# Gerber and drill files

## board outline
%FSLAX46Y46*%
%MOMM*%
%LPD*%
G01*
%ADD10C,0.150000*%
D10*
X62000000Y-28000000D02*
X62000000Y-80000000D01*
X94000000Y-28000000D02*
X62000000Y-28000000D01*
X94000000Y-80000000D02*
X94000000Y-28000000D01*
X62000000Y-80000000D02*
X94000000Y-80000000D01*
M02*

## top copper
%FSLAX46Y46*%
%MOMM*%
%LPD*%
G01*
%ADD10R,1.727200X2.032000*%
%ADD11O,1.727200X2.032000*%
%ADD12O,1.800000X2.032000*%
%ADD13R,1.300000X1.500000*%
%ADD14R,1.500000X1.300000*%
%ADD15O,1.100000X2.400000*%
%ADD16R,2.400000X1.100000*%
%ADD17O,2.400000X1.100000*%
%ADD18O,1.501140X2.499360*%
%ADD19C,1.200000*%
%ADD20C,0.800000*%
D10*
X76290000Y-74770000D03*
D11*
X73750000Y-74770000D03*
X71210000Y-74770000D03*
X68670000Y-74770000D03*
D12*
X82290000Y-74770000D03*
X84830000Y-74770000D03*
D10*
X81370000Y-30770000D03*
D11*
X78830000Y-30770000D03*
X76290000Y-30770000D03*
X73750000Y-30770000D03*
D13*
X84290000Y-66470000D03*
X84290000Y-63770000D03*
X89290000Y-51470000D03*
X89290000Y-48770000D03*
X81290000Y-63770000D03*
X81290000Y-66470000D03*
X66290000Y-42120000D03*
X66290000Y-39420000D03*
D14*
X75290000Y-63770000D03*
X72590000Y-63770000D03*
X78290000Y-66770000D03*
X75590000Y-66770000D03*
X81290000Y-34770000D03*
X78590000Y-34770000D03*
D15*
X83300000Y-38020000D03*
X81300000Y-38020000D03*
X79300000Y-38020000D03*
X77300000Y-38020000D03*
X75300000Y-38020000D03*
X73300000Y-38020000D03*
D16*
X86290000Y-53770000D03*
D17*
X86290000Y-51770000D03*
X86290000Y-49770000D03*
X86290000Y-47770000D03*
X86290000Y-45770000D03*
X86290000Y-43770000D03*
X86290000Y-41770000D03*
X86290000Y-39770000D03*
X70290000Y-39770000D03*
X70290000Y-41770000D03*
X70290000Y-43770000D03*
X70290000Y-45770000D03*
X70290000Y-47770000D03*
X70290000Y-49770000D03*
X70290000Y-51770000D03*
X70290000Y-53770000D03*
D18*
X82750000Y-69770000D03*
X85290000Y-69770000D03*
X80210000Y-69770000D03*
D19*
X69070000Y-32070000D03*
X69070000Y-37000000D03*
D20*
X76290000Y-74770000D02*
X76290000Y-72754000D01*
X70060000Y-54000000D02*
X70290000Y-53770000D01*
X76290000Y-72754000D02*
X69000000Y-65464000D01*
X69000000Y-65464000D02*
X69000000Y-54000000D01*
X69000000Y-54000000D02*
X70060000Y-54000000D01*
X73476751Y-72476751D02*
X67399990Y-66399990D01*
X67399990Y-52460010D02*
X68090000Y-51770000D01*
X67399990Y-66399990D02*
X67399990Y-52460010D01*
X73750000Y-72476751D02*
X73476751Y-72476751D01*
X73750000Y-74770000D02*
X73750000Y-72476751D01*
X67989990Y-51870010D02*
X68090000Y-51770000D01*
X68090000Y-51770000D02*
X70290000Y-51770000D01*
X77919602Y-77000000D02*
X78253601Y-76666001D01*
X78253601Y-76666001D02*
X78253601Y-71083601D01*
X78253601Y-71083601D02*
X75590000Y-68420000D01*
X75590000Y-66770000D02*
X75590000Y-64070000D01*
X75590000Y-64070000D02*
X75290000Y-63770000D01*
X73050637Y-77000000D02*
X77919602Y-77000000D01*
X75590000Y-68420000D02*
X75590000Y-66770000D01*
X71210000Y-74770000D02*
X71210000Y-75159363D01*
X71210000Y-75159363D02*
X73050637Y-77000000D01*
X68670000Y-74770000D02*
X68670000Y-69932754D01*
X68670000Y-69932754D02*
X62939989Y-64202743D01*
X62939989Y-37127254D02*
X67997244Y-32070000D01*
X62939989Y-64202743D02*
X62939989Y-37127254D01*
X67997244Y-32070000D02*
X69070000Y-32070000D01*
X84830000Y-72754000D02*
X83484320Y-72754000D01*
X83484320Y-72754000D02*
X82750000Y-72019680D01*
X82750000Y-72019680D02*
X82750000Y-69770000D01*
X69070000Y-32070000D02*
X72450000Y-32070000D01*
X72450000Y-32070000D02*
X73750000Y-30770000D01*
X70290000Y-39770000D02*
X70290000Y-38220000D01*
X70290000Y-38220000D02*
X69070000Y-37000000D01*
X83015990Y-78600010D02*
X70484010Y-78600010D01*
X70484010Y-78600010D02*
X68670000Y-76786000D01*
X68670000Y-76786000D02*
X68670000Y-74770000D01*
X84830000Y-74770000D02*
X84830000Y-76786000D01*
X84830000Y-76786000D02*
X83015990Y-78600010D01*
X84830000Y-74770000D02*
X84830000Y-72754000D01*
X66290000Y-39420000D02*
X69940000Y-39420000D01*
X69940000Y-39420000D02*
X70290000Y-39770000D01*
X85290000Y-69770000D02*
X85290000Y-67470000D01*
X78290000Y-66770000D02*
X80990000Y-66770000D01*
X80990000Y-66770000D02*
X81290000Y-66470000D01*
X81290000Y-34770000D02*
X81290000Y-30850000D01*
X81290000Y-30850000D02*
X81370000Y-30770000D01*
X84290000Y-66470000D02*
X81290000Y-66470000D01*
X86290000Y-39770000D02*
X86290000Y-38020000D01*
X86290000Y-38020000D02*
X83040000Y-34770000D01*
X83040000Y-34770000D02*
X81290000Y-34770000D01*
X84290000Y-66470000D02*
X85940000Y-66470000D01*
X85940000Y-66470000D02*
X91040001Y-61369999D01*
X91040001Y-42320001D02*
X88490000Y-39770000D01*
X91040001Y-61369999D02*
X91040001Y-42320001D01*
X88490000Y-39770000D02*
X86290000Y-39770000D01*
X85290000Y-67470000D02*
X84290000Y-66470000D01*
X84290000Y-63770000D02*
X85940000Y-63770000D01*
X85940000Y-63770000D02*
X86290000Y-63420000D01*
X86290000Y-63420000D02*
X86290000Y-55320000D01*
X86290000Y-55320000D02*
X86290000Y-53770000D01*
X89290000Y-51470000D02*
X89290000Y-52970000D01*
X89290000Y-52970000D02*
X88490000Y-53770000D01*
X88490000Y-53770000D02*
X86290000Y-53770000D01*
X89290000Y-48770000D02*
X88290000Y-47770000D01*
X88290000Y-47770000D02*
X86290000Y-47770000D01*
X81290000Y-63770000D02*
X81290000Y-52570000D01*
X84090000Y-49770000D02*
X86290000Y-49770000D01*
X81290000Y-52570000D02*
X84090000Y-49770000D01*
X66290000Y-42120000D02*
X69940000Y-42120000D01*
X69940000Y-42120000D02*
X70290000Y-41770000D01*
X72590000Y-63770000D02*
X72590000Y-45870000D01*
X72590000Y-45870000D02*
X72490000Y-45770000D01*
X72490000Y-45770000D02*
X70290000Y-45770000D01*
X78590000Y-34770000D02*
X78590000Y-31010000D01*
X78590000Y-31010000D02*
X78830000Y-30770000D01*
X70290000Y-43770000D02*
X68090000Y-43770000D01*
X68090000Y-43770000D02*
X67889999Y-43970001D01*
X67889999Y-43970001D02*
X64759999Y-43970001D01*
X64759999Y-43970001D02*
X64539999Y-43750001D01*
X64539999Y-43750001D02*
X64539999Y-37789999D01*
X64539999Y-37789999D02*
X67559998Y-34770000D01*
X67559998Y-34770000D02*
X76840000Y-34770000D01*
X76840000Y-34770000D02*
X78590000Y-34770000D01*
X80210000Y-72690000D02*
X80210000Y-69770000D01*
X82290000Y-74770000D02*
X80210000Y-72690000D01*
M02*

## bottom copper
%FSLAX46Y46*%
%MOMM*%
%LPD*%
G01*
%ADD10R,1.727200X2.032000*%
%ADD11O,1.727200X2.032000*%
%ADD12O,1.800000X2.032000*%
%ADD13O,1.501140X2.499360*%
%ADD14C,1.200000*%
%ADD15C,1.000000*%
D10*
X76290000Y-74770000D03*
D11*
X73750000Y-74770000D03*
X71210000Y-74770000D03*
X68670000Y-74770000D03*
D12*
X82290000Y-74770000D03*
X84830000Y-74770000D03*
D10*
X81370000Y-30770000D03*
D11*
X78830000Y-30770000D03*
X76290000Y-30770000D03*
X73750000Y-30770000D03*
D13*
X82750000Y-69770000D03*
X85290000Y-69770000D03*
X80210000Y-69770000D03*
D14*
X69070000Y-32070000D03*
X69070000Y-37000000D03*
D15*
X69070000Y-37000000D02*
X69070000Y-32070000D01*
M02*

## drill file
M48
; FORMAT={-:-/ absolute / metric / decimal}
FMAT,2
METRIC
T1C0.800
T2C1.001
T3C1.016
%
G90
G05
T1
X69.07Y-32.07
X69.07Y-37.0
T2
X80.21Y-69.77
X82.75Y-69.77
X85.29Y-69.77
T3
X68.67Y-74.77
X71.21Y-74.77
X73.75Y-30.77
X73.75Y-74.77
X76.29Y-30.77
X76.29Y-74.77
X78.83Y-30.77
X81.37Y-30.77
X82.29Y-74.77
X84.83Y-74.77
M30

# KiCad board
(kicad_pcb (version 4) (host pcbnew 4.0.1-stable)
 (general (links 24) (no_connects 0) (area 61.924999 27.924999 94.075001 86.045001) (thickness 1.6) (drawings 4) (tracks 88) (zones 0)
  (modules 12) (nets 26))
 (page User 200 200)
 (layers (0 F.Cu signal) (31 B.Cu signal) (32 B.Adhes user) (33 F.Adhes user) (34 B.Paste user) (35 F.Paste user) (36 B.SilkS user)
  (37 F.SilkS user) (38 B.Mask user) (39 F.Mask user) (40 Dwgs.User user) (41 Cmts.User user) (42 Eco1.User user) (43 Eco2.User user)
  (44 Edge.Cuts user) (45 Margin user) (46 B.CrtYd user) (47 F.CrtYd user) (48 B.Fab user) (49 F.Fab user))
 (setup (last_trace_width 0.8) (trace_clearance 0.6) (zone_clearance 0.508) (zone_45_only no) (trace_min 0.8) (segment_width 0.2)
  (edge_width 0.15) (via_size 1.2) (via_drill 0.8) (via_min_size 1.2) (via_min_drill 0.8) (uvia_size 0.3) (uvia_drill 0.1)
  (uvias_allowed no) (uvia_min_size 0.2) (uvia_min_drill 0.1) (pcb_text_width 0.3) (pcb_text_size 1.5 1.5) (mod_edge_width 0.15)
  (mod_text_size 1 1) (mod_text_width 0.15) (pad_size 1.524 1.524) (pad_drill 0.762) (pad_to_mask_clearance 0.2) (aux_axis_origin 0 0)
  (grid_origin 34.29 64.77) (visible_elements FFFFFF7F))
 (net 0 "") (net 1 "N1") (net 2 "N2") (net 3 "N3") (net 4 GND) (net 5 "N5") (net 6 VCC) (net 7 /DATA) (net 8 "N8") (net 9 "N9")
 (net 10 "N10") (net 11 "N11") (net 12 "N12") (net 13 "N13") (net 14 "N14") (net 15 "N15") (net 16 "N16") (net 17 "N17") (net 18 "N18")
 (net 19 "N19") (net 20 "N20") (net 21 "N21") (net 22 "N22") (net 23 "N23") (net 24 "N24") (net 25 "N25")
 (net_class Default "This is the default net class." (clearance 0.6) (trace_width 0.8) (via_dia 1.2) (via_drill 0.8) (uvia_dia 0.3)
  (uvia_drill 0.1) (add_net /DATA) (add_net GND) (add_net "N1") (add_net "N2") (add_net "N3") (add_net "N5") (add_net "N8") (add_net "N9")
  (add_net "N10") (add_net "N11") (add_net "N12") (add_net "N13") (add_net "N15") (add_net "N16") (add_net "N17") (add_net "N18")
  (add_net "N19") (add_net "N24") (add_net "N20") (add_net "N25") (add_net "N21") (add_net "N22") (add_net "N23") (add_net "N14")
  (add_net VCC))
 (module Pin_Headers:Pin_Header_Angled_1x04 (layer F.Cu) (at 76.29 74.77 270)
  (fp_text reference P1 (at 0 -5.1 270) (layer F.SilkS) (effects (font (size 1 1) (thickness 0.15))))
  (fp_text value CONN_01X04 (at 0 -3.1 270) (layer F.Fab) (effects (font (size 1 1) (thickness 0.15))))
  (pad 1 thru_hole rect (at 0 0 270) (size 2.032 1.7272) (drill 1.016) (layers *.Cu *.Mask F.SilkS) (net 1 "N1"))
  (pad 2 thru_hole oval (at 0 2.54 270) (size 2.032 1.7272) (drill 1.016) (layers *.Cu *.Mask F.SilkS) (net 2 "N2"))
  (pad 3 thru_hole oval (at 0 5.08 270) (size 2.032 1.7272) (drill 1.016) (layers *.Cu *.Mask F.SilkS) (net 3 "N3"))
  (pad 4 thru_hole oval (at 0 7.62 270) (size 2.032 1.7272) (drill 1.016) (layers *.Cu *.Mask F.SilkS) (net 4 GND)))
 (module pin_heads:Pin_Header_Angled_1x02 (layer F.Cu) (at 84.83 74.77 270)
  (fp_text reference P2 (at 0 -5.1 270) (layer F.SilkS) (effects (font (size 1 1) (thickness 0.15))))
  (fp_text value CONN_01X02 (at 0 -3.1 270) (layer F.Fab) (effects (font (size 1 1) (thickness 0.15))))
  (pad 2 thru_hole oval (at 0 2.54 270) (size 2.032 1.8) (drill 1.016) (layers *.Cu *.Mask F.SilkS) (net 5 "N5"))
  (pad 1 thru_hole oval (at 0 0 270) (size 2.032 1.8) (drill 1.016) (layers *.Cu *.Mask F.SilkS) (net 4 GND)))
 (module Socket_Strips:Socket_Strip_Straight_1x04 (layer F.Cu) (at 81.37 30.77 180)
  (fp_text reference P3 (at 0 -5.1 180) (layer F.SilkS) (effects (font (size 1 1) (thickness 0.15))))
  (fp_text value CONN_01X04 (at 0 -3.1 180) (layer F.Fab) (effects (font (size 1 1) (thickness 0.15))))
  (pad 1 thru_hole rect (at 0 0 180) (size 1.7272 2.032) (drill 1.016) (layers *.Cu *.Mask F.SilkS) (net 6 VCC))
  (pad 2 thru_hole oval (at 2.54 0 180) (size 1.7272 2.032) (drill 1.016) (layers *.Cu *.Mask F.SilkS) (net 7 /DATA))
  (pad 3 thru_hole oval (at 5.08 0 180) (size 1.7272 2.032) (drill 1.016) (layers *.Cu *.Mask F.SilkS) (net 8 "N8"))
  (pad 4 thru_hole oval (at 7.62 0 180) (size 1.7272 2.032) (drill 1.016) (layers *.Cu *.Mask F.SilkS) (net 4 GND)))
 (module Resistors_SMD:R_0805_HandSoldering (layer F.Cu) (at 84.29 65.12 90)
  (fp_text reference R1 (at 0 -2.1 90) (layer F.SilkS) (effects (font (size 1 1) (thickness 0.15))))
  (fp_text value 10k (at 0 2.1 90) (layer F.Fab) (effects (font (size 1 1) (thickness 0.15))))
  (pad 1 smd rect (at -1.35 0 90) (size 1.5 1.3) (layers F.Cu F.Paste F.Mask) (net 6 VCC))
  (pad 2 smd rect (at 1.35 0 90) (size 1.5 1.3) (layers F.Cu F.Paste F.Mask) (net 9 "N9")))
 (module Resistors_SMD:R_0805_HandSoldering (layer F.Cu) (at 89.29 50.12 90)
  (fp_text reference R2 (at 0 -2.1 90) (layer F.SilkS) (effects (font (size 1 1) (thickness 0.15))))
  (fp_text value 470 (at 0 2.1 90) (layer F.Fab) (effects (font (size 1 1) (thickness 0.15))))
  (pad 1 smd rect (at -1.35 0 90) (size 1.5 1.3) (layers F.Cu F.Paste F.Mask) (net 9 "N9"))
  (pad 2 smd rect (at 1.35 0 90) (size 1.5 1.3) (layers F.Cu F.Paste F.Mask) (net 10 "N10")))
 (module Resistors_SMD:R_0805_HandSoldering (layer F.Cu) (at 81.29 65.12 270)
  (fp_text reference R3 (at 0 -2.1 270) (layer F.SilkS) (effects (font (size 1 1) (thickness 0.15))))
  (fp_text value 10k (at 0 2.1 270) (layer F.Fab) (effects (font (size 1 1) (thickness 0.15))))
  (pad 1 smd rect (at -1.35 0 270) (size 1.5 1.3) (layers F.Cu F.Paste F.Mask) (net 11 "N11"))
  (pad 2 smd rect (at 1.35 0 270) (size 1.5 1.3) (layers F.Cu F.Paste F.Mask) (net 6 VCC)))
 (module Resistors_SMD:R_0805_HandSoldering (layer F.Cu) (at 66.29 40.77 90)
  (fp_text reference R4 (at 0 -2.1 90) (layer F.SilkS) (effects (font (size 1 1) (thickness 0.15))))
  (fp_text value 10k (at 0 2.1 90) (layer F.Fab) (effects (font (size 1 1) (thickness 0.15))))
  (pad 1 smd rect (at -1.35 0 90) (size 1.5 1.3) (layers F.Cu F.Paste F.Mask) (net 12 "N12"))
  (pad 2 smd rect (at 1.35 0 90) (size 1.5 1.3) (layers F.Cu F.Paste F.Mask) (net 4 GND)))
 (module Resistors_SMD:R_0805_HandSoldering (layer F.Cu) (at 73.94 63.77 180)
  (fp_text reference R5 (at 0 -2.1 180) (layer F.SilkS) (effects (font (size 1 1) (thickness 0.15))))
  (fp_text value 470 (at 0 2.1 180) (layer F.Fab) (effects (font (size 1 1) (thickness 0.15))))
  (pad 1 smd rect (at -1.35 0 180) (size 1.5 1.3) (layers F.Cu F.Paste F.Mask) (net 3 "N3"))
  (pad 2 smd rect (at 1.35 0 180) (size 1.5 1.3) (layers F.Cu F.Paste F.Mask) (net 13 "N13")))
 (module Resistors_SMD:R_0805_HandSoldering (layer F.Cu) (at 76.94 66.77 180)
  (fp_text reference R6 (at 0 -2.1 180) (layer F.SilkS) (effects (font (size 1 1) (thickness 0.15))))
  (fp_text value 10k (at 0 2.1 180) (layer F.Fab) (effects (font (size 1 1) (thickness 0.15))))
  (pad 1 smd rect (at -1.35 0 180) (size 1.5 1.3) (layers F.Cu F.Paste F.Mask) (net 6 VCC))
  (pad 2 smd rect (at 1.35 0 180) (size 1.5 1.3) (layers F.Cu F.Paste F.Mask) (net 3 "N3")))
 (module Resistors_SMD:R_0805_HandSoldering (layer F.Cu) (at 79.94 34.77 180)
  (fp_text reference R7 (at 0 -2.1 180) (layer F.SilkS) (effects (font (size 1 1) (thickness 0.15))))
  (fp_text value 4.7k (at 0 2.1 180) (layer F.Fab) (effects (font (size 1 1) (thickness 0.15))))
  (pad 1 smd rect (at -1.35 0 180) (size 1.5 1.3) (layers F.Cu F.Paste F.Mask) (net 6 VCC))
  (pad 2 smd rect (at 1.35 0 180) (size 1.5 1.3) (layers F.Cu F.Paste F.Mask) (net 7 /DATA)))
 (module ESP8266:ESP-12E (layer F.Cu) (at 86.29 53.77 180)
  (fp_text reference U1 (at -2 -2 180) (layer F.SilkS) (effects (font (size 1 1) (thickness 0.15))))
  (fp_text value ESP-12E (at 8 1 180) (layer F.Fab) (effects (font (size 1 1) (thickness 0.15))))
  (pad 9 smd oval (at 2.99 15.75 270) (size 2.4 1.1) (layers F.Cu F.Paste F.Mask) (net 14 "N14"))
  (pad 10 smd oval (at 4.99 15.75 270) (size 2.4 1.1) (layers F.Cu F.Paste F.Mask) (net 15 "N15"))
  (pad 11 smd oval (at 6.99 15.75 270) (size 2.4 1.1) (layers F.Cu F.Paste F.Mask) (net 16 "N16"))
  (pad 12 smd oval (at 8.99 15.75 270) (size 2.4 1.1) (layers F.Cu F.Paste F.Mask) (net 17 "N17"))
  (pad 13 smd oval (at 10.99 15.75 270) (size 2.4 1.1) (layers F.Cu F.Paste F.Mask) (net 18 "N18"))
  (pad 14 smd oval (at 12.99 15.75 270) (size 2.4 1.1) (layers F.Cu F.Paste F.Mask) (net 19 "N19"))
  (pad 1 smd rect (at 0 0 180) (size 2.4 1.1) (layers F.Cu F.Paste F.Mask) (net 9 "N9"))
  (pad 2 smd oval (at 0 2 180) (size 2.4 1.1) (layers F.Cu F.Paste F.Mask) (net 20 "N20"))
  (pad 3 smd oval (at 0 4 180) (size 2.4 1.1) (layers F.Cu F.Paste F.Mask) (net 11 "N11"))
  (pad 4 smd oval (at 0 6 180) (size 2.4 1.1) (layers F.Cu F.Paste F.Mask) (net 10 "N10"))
  (pad 5 smd oval (at 0 8 180) (size 2.4 1.1) (layers F.Cu F.Paste F.Mask) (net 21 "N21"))
  (pad 6 smd oval (at 0 10 180) (size 2.4 1.1) (layers F.Cu F.Paste F.Mask) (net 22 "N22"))
  (pad 7 smd oval (at 0 12 180) (size 2.4 1.1) (layers F.Cu F.Paste F.Mask) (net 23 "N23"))
  (pad 8 smd oval (at 0 14 180) (size 2.4 1.1) (layers F.Cu F.Paste F.Mask) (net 6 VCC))
  (pad 15 smd oval (at 16 14 180) (size 2.4 1.1) (layers F.Cu F.Paste F.Mask) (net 4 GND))
  (pad 16 smd oval (at 16 12 180) (size 2.4 1.1) (layers F.Cu F.Paste F.Mask) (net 12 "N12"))
  (pad 17 smd oval (at 16 10 180) (size 2.4 1.1) (layers F.Cu F.Paste F.Mask) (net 7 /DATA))
  (pad 18 smd oval (at 16 8 180) (size 2.4 1.1) (layers F.Cu F.Paste F.Mask) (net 13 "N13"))
  (pad 19 smd oval (at 16 6 180) (size 2.4 1.1) (layers F.Cu F.Paste F.Mask) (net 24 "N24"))
  (pad 20 smd oval (at 16 4 180) (size 2.4 1.1) (layers F.Cu F.Paste F.Mask) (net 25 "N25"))
  (pad 21 smd oval (at 16 2 180) (size 2.4 1.1) (layers F.Cu F.Paste F.Mask) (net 2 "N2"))
  (pad 22 smd oval (at 16 0 180) (size 2.4 1.1) (layers F.Cu F.Paste F.Mask) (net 1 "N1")))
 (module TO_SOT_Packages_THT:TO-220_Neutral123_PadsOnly (layer F.Cu) (at 82.75 69.77 180)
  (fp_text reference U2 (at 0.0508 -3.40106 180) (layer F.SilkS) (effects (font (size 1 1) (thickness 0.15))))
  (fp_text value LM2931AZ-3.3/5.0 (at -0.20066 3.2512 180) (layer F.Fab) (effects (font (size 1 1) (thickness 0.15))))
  (pad 2 thru_hole oval (at 0 0 270) (size 2.49936 1.50114) (drill 1.00076) (layers *.Cu *.Mask F.SilkS) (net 4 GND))
  (pad 1 thru_hole oval (at -2.54 0 270) (size 2.49936 1.50114) (drill 1.00076) (layers *.Cu *.Mask F.SilkS) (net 6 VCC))
  (pad 3 thru_hole oval (at 2.54 0 270) (size 2.49936 1.50114) (drill 1.00076) (layers *.Cu *.Mask F.SilkS) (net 5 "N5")))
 (gr_line (start 62 28) (end 62 80) (layer Edge.Cuts) (width 0.15))
 (gr_line (start 94 28) (end 62 28) (layer Edge.Cuts) (width 0.15))
 (gr_line (start 94 80) (end 94 28) (layer Edge.Cuts) (width 0.15))
 (gr_line (start 62 80) (end 94 80) (layer Edge.Cuts) (width 0.15))
 (segment (start 76.29 74.77) (end 76.29 72.754) (width 0.8) (layer F.Cu) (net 1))
 (segment (start 70.06 54) (end 70.29 53.77) (width 0.8) (layer F.Cu) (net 1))
 (segment (start 76.29 72.754) (end 69 65.464) (width 0.8) (layer F.Cu) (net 1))
 (segment (start 69 65.464) (end 69 54) (width 0.8) (layer F.Cu) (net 1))
 (segment (start 69 54) (end 70.06 54) (width 0.8) (layer F.Cu) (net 1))
 (segment (start 73.476751 72.476751) (end 67.39999 66.39999) (width 0.8) (layer F.Cu) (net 2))
 (segment (start 67.39999 52.46001) (end 68.09 51.77) (width 0.8) (layer F.Cu) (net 2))
 (segment (start 67.39999 66.39999) (end 67.39999 52.46001) (width 0.8) (layer F.Cu) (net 2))
 (segment (start 73.75 72.476751) (end 73.476751 72.476751) (width 0.8) (layer F.Cu) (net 2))
 (segment (start 73.75 74.77) (end 73.75 72.476751) (width 0.8) (layer F.Cu) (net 2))
 (segment (start 67.98999 51.87001) (end 68.09 51.77) (width 0.8) (layer F.Cu) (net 2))
 (segment (start 68.09 51.77) (end 70.29 51.77) (width 0.8) (layer F.Cu) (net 2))
 (segment (start 77.919602 77) (end 78.253601 76.666001) (width 0.8) (layer F.Cu) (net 3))
 (segment (start 78.253601 76.666001) (end 78.253601 71.083601) (width 0.8) (layer F.Cu) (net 3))
 (segment (start 78.253601 71.083601) (end 75.59 68.42) (width 0.8) (layer F.Cu) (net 3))
 (segment (start 75.59 66.77) (end 75.59 64.07) (width 0.8) (layer F.Cu) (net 3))
 (segment (start 75.59 64.07) (end 75.29 63.77) (width 0.8) (layer F.Cu) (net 3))
 (segment (start 73.050637 77) (end 77.919602 77) (width 0.8) (layer F.Cu) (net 3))
 (segment (start 75.59 68.42) (end 75.59 66.77) (width 0.8) (layer F.Cu) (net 3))
 (segment (start 71.21 74.77) (end 71.21 75.159363) (width 0.8) (layer F.Cu) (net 3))
 (segment (start 71.21 75.159363) (end 73.050637 77) (width 0.8) (layer F.Cu) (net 3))
 (segment (start 68.67 74.77) (end 68.67 69.932754) (width 0.8) (layer F.Cu) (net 4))
 (segment (start 68.67 69.932754) (end 62.939989 64.202743) (width 0.8) (layer F.Cu) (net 4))
 (segment (start 62.939989 37.127254) (end 67.997244 32.07) (width 0.8) (layer F.Cu) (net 4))
 (segment (start 62.939989 64.202743) (end 62.939989 37.127254) (width 0.8) (layer F.Cu) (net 4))
 (segment (start 67.997244 32.07) (end 69.07 32.07) (width 0.8) (layer F.Cu) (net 4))
 (segment (start 84.83 72.754) (end 83.48432 72.754) (width 0.8) (layer F.Cu) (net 4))
 (segment (start 83.48432 72.754) (end 82.75 72.01968) (width 0.8) (layer F.Cu) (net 4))
 (segment (start 82.75 72.01968) (end 82.75 69.77) (width 0.8) (layer F.Cu) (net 4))
 (segment (start 69.07 32.07) (end 72.45 32.07) (width 0.8) (layer F.Cu) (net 4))
 (segment (start 72.45 32.07) (end 73.75 30.77) (width 0.8) (layer F.Cu) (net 4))
 (via (at 69.07 32.07) (size 1.2) (drill 0.8) (layers F.Cu B.Cu) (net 4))
 (segment (start 69.07 37) (end 69.07 32.07) (width 1) (layer B.Cu) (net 4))
 (via (at 69.07 37) (size 1.2) (drill 0.8) (layers F.Cu B.Cu) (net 4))
 (segment (start 70.29 39.77) (end 70.29 38.22) (width 0.8) (layer F.Cu) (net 4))
 (segment (start 70.29 38.22) (end 69.07 37) (width 0.8) (layer F.Cu) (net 4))
 (segment (start 83.01599 78.60001) (end 70.48401 78.60001) (width 0.8) (layer F.Cu) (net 4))
 (segment (start 70.48401 78.60001) (end 68.67 76.786) (width 0.8) (layer F.Cu) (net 4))
 (segment (start 68.67 76.786) (end 68.67 74.77) (width 0.8) (layer F.Cu) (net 4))
 (segment (start 84.83 74.77) (end 84.83 76.786) (width 0.8) (layer F.Cu) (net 4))
 (segment (start 84.83 76.786) (end 83.01599 78.60001) (width 0.8) (layer F.Cu) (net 4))
 (segment (start 84.83 74.77) (end 84.83 72.754) (width 0.8) (layer F.Cu) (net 4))
 (segment (start 66.29 39.42) (end 69.94 39.42) (width 0.8) (layer F.Cu) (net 4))
 (segment (start 69.94 39.42) (end 70.29 39.77) (width 0.8) (layer F.Cu) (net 4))
 (segment (start 85.29 69.77) (end 85.29 67.47) (width 0.8) (layer F.Cu) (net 6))
 (segment (start 78.29 66.77) (end 80.99 66.77) (width 0.8) (layer F.Cu) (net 6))
 (segment (start 80.99 66.77) (end 81.29 66.47) (width 0.8) (layer F.Cu) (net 6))
 (segment (start 81.29 34.77) (end 81.29 30.85) (width 0.8) (layer F.Cu) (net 6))
 (segment (start 81.29 30.85) (end 81.37 30.77) (width 0.8) (layer F.Cu) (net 6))
 (segment (start 84.29 66.47) (end 81.29 66.47) (width 0.8) (layer F.Cu) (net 6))
 (segment (start 86.29 39.77) (end 86.29 38.02) (width 0.8) (layer F.Cu) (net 6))
 (segment (start 86.29 38.02) (end 83.04 34.77) (width 0.8) (layer F.Cu) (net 6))
 (segment (start 83.04 34.77) (end 81.29 34.77) (width 0.8) (layer F.Cu) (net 6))
 (segment (start 84.29 66.47) (end 85.94 66.47) (width 0.8) (layer F.Cu) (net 6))
 (segment (start 85.94 66.47) (end 91.040001 61.369999) (width 0.8) (layer F.Cu) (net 6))
 (segment (start 91.040001 42.320001) (end 88.49 39.77) (width 0.8) (layer F.Cu) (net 6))
 (segment (start 91.040001 61.369999) (end 91.040001 42.320001) (width 0.8) (layer F.Cu) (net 6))
 (segment (start 88.49 39.77) (end 86.29 39.77) (width 0.8) (layer F.Cu) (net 6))
 (segment (start 85.29 67.47) (end 84.29 66.47) (width 0.8) (layer F.Cu) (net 6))
 (segment (start 84.29 63.77) (end 85.94 63.77) (width 0.8) (layer F.Cu) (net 9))
 (segment (start 85.94 63.77) (end 86.29 63.42) (width 0.8) (layer F.Cu) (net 9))
 (segment (start 86.29 63.42) (end 86.29 55.32) (width 0.8) (layer F.Cu) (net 9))
 (segment (start 86.29 55.32) (end 86.29 53.77) (width 0.8) (layer F.Cu) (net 9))
 (segment (start 89.29 51.47) (end 89.29 52.97) (width 0.8) (layer F.Cu) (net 9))
 (segment (start 89.29 52.97) (end 88.49 53.77) (width 0.8) (layer F.Cu) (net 9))
 (segment (start 88.49 53.77) (end 86.29 53.77) (width 0.8) (layer F.Cu) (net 9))
 (segment (start 89.29 48.77) (end 88.29 47.77) (width 0.8) (layer F.Cu) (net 10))
 (segment (start 88.29 47.77) (end 86.29 47.77) (width 0.8) (layer F.Cu) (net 10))
 (segment (start 81.29 63.77) (end 81.29 52.57) (width 0.8) (layer F.Cu) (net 11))
 (segment (start 84.09 49.77) (end 86.29 49.77) (width 0.8) (layer F.Cu) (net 11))
 (segment (start 81.29 52.57) (end 84.09 49.77) (width 0.8) (layer F.Cu) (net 11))
 (segment (start 66.29 42.12) (end 69.94 42.12) (width 0.8) (layer F.Cu) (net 12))
 (segment (start 69.94 42.12) (end 70.29 41.77) (width 0.8) (layer F.Cu) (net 12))
 (segment (start 72.59 63.77) (end 72.59 45.87) (width 0.8) (layer F.Cu) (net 13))
 (segment (start 72.59 45.87) (end 72.49 45.77) (width 0.8) (layer F.Cu) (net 13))
 (segment (start 72.49 45.77) (end 70.29 45.77) (width 0.8) (layer F.Cu) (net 13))
 (segment (start 78.59 34.77) (end 78.59 31.01) (width 0.8) (layer F.Cu) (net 7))
 (segment (start 78.59 31.01) (end 78.83 30.77) (width 0.8) (layer F.Cu) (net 7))
 (segment (start 70.29 43.77) (end 68.09 43.77) (width 0.8) (layer F.Cu) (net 7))
 (segment (start 68.09 43.77) (end 67.889999 43.970001) (width 0.8) (layer F.Cu) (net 7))
 (segment (start 67.889999 43.970001) (end 64.759999 43.970001) (width 0.8) (layer F.Cu) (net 7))
 (segment (start 64.759999 43.970001) (end 64.539999 43.750001) (width 0.8) (layer F.Cu) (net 7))
 (segment (start 64.539999 43.750001) (end 64.539999 37.789999) (width 0.8) (layer F.Cu) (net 7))
 (segment (start 64.539999 37.789999) (end 67.559998 34.77) (width 0.8) (layer F.Cu) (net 7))
 (segment (start 67.559998 34.77) (end 76.84 34.77) (width 0.8) (layer F.Cu) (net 7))
 (segment (start 76.84 34.77) (end 78.59 34.77) (width 0.8) (layer F.Cu) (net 7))
 (segment (start 80.21 72.69) (end 80.21 69.77) (width 0.8) (layer F.Cu) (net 5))
 (segment (start 82.29 74.77) (end 80.21 72.69) (width 0.8) (layer F.Cu) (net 5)))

